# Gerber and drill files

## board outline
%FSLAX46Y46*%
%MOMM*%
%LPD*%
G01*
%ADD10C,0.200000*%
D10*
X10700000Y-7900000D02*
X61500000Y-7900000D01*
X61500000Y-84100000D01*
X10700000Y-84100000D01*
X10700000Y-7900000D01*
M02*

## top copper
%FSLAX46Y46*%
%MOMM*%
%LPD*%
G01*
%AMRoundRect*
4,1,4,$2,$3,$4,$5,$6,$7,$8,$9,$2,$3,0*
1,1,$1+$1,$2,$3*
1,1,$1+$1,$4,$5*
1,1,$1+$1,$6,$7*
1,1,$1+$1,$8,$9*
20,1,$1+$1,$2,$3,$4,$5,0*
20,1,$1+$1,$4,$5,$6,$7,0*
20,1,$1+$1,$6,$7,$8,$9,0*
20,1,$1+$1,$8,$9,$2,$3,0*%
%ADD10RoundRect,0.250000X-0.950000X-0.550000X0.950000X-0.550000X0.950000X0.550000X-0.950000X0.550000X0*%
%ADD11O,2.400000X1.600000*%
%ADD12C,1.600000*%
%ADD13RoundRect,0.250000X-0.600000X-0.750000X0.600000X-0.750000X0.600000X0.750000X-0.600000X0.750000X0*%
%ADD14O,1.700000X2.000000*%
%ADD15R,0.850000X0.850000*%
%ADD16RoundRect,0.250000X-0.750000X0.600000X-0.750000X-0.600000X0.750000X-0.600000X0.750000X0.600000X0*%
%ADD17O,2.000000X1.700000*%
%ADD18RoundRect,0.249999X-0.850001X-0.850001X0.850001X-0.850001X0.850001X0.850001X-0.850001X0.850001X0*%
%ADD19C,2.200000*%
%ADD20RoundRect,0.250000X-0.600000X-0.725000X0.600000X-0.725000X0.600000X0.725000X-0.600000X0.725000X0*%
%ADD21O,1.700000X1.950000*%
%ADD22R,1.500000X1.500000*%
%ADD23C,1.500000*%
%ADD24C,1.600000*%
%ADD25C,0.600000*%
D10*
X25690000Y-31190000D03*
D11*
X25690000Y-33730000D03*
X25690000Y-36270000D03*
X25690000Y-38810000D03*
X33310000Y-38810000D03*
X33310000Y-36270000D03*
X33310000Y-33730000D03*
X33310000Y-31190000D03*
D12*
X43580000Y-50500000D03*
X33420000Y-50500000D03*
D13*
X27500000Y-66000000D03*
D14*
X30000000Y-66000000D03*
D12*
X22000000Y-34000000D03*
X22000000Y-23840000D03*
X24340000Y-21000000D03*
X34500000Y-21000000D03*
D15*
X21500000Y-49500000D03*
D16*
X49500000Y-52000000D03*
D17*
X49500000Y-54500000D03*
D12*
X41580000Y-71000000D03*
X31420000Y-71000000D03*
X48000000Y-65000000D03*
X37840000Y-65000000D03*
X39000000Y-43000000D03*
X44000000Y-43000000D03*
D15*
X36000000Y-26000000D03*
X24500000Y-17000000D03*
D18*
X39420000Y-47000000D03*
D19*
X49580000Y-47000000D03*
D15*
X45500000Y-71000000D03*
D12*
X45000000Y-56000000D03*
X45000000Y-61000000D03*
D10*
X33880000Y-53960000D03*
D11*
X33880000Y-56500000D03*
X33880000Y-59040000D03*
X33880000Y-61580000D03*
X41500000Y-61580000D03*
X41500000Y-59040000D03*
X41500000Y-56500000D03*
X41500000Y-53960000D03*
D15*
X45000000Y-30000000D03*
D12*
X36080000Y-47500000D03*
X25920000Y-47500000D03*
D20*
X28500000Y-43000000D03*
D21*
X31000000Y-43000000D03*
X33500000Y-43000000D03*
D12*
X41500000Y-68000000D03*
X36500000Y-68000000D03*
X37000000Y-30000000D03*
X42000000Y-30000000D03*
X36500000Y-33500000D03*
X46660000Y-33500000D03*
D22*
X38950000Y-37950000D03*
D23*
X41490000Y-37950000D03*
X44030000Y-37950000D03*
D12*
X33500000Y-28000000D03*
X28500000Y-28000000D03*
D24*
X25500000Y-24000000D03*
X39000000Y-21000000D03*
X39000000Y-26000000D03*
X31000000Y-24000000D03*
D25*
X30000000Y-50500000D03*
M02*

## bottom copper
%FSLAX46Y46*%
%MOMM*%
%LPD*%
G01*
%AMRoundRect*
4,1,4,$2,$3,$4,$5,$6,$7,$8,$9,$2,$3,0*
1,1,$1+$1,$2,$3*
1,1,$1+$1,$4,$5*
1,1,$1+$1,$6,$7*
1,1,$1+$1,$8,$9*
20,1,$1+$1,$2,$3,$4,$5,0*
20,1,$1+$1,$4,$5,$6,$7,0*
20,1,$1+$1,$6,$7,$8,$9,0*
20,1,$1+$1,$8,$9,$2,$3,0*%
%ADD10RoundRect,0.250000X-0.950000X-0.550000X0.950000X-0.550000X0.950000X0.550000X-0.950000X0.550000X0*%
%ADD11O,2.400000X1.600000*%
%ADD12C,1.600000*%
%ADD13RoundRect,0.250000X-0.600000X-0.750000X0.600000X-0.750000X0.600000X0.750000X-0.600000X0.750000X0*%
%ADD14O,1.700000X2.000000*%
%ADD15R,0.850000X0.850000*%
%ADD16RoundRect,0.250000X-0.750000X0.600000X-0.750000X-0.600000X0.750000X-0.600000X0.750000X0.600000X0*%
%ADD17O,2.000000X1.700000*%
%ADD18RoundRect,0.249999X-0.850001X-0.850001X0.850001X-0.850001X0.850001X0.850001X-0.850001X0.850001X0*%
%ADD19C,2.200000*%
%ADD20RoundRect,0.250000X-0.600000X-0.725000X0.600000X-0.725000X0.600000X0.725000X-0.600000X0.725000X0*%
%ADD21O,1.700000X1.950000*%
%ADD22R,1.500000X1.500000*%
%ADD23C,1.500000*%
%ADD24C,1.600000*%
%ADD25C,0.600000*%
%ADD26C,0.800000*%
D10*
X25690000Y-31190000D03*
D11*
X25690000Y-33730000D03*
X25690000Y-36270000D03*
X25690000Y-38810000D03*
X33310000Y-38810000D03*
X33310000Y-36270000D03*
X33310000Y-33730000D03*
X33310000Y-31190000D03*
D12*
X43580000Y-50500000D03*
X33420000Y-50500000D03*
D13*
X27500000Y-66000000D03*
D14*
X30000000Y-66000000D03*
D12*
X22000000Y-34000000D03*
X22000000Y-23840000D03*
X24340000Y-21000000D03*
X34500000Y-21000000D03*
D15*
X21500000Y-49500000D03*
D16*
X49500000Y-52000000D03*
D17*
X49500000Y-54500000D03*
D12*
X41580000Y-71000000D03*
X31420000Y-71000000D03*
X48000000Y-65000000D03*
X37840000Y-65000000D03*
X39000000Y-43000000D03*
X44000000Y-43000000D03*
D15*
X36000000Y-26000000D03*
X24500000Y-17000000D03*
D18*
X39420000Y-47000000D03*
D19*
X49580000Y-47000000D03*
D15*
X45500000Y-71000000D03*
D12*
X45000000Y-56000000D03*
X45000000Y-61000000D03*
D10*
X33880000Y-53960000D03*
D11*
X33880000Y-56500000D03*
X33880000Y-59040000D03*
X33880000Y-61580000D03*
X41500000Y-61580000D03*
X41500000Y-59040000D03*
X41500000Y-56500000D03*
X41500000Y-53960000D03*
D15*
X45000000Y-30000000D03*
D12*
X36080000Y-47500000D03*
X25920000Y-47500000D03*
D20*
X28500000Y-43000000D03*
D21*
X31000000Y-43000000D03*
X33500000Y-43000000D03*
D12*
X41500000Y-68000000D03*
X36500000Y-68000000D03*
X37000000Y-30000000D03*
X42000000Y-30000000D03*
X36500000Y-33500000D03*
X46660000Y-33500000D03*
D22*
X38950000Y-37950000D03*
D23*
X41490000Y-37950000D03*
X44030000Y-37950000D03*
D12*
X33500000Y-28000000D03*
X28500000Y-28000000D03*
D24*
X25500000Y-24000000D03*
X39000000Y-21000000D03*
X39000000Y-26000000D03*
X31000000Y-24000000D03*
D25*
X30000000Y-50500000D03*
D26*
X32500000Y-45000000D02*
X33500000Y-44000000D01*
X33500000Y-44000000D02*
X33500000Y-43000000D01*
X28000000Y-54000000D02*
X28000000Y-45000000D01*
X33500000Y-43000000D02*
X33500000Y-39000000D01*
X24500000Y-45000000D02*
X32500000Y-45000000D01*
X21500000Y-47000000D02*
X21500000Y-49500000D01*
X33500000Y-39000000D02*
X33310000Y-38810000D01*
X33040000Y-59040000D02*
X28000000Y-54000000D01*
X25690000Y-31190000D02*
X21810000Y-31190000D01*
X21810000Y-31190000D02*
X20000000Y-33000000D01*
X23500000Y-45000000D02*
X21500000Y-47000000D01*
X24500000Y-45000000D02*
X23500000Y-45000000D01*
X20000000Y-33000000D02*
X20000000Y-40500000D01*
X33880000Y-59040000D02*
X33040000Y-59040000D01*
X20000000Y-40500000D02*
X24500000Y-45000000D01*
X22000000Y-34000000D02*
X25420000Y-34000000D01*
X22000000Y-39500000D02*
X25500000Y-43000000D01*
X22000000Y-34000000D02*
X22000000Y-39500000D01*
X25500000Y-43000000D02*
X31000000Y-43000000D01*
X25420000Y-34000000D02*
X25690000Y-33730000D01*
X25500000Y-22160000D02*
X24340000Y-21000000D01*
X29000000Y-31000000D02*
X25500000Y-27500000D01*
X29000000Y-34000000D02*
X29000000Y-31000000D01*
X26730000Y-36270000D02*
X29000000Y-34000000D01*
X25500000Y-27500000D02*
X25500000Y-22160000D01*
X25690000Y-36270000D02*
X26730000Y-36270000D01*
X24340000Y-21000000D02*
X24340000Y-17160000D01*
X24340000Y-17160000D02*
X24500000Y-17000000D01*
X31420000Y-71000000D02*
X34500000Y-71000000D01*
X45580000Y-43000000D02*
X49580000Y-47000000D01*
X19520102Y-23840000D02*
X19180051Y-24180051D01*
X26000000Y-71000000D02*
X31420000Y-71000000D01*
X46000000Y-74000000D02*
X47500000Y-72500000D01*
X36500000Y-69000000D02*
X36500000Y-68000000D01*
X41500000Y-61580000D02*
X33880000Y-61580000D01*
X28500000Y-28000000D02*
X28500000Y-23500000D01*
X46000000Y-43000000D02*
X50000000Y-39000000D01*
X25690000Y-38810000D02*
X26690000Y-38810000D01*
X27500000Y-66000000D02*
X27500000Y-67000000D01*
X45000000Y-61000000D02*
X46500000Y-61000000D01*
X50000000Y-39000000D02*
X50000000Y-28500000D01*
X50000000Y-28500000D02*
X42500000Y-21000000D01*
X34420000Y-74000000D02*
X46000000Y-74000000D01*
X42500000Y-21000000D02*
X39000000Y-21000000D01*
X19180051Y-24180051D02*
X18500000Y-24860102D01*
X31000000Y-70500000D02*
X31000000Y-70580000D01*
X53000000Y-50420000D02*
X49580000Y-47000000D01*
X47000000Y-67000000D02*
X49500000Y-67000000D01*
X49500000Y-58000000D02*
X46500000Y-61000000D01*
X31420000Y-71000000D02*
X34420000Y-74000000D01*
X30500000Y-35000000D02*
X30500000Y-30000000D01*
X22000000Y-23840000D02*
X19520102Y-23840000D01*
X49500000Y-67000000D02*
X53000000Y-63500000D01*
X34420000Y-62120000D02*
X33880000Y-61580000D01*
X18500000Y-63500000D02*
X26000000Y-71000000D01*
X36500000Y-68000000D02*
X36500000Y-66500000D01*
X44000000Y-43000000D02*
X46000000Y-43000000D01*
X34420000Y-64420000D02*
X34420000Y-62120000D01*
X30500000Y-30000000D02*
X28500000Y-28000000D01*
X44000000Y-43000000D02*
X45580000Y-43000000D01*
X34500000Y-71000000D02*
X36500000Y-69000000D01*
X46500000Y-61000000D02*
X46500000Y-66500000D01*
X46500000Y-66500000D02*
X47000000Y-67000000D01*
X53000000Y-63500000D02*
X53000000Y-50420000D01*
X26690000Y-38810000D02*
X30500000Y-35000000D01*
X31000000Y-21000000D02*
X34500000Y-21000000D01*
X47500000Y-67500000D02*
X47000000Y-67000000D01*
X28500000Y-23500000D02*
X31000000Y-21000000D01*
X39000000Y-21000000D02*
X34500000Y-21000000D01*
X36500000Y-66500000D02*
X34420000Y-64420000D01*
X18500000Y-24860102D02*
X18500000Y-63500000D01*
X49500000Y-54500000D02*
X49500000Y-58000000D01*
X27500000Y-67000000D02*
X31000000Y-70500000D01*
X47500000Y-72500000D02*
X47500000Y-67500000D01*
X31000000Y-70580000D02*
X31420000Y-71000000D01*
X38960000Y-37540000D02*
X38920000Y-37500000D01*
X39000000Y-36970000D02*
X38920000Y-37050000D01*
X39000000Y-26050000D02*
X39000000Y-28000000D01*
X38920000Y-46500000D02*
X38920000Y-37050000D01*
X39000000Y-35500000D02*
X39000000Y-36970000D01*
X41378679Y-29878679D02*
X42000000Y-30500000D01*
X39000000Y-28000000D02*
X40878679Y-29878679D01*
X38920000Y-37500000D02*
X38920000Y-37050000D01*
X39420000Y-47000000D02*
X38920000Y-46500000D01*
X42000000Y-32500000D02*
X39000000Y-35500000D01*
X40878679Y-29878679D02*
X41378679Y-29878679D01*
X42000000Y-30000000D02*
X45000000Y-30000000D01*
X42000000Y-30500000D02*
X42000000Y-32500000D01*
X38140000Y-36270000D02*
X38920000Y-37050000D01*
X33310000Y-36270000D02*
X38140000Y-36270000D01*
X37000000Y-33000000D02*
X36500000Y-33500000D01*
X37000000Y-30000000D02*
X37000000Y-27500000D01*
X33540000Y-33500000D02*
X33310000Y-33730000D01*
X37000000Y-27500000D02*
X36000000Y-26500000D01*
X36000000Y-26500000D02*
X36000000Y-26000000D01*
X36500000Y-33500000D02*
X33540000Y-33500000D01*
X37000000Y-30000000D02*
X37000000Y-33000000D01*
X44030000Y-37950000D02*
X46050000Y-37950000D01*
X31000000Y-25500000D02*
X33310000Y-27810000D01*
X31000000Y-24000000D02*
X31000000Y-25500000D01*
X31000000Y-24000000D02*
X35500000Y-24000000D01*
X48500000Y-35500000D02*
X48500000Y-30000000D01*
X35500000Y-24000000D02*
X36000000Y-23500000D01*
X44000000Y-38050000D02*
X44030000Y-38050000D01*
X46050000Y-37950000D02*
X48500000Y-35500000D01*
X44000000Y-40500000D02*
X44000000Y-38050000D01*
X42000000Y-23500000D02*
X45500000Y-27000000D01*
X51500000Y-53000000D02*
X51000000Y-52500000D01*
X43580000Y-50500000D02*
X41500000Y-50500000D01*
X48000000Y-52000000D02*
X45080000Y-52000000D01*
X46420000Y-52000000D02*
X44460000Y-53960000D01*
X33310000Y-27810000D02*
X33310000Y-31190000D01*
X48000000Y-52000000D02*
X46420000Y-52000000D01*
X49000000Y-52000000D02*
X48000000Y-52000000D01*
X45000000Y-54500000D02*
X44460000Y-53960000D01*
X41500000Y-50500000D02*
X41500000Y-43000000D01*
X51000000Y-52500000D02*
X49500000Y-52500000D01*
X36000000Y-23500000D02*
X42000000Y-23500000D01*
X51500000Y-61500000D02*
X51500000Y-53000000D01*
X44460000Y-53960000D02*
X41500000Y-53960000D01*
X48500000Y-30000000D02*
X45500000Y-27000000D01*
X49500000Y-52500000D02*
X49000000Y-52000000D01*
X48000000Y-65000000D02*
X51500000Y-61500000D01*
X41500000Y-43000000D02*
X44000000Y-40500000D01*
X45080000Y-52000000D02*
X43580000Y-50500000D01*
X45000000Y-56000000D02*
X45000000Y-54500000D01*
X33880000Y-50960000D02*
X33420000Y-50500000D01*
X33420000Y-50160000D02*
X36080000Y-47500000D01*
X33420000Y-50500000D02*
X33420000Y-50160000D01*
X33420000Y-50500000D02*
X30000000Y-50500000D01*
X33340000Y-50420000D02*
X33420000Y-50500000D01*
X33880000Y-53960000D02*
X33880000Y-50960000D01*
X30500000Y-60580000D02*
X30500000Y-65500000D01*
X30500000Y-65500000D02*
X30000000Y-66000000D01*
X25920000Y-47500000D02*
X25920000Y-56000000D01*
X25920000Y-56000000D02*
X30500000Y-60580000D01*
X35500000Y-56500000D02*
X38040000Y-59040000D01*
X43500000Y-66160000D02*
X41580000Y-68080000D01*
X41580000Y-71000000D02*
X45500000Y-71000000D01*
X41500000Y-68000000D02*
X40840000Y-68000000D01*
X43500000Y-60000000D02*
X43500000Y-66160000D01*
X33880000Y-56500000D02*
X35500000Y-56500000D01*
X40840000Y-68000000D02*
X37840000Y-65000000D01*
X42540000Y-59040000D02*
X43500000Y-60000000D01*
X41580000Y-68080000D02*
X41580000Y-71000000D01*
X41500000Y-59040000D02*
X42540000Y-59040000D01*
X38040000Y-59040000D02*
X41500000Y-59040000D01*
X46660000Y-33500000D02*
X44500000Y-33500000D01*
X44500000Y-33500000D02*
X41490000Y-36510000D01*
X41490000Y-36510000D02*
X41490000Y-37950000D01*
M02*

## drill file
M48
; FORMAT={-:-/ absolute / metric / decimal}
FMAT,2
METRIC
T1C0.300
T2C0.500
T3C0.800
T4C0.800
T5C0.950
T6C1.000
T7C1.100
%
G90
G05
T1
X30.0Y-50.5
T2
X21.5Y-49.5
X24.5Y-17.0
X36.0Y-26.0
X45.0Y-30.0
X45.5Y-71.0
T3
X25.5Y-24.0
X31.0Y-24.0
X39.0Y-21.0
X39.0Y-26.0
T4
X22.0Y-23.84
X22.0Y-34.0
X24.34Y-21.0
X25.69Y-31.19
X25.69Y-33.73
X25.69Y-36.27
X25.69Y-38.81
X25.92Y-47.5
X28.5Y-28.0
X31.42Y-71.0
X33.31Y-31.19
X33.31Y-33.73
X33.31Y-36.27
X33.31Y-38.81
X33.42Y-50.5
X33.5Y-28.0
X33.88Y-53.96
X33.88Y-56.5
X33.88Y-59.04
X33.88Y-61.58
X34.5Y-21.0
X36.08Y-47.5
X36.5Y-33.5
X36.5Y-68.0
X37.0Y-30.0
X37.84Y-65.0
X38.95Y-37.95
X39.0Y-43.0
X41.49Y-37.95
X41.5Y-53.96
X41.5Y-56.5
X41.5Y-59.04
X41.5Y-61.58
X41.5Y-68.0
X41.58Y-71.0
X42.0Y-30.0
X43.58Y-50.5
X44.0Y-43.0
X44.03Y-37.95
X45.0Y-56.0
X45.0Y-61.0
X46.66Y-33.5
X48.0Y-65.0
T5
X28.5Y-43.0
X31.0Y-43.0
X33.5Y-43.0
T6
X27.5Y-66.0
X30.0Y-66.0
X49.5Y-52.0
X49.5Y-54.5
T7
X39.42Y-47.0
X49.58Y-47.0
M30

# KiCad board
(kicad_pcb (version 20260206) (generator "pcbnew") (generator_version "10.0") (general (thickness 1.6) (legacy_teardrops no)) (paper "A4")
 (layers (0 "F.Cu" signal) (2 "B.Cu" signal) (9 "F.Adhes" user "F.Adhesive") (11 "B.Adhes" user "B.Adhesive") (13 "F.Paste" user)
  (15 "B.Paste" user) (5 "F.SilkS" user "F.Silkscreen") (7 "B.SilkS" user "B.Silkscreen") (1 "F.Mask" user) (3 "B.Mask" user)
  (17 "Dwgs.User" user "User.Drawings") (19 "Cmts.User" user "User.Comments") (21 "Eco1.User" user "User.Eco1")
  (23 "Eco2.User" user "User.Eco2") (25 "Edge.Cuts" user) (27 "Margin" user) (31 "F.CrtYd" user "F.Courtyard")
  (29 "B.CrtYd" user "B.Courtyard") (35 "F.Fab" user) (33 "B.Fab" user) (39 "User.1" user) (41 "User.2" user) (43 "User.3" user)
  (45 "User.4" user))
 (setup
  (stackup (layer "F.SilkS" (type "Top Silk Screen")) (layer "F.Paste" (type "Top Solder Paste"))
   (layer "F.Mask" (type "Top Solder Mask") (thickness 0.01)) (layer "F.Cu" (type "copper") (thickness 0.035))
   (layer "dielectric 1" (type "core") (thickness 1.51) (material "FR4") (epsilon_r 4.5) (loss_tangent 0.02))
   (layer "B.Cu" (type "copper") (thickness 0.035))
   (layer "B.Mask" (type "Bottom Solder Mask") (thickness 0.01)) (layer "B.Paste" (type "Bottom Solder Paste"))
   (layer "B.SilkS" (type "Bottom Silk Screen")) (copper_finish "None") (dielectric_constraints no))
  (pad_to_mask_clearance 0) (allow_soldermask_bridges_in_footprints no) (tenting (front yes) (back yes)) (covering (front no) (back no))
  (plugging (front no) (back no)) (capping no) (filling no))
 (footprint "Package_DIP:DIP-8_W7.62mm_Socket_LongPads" (layer "F.Cu") (at 25.69 31.19)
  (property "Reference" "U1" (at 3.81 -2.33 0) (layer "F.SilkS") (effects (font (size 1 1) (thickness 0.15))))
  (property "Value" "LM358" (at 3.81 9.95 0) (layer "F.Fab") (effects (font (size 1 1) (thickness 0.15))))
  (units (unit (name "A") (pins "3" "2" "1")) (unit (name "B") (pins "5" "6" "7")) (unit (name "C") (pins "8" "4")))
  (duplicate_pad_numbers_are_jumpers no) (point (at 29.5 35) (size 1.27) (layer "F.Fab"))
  (pad "1" thru_hole roundrect (at 0 0) (size 2.4 1.6) (drill 0.8) (layers "*.Cu" "*.Mask") (remove_unused_layers no)
   (roundrect_rratio 0.15625) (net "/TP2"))
  (pad "2" thru_hole oval (at 0 2.54) (size 2.4 1.6) (drill 0.8) (layers "*.Cu" "*.Mask") (remove_unused_layers no) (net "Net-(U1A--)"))
  (pad "3" thru_hole oval (at 0 5.08) (size 2.4 1.6) (drill 0.8) (layers "*.Cu" "*.Mask") (remove_unused_layers no) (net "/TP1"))
  (pad "4" thru_hole oval (at 0 7.62) (size 2.4 1.6) (drill 0.8) (layers "*.Cu" "*.Mask") (remove_unused_layers no) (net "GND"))
  (pad "5" thru_hole oval (at 7.62 7.62) (size 2.4 1.6) (drill 0.8) (layers "*.Cu" "*.Mask") (remove_unused_layers no) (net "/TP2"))
  (pad "6" thru_hole oval (at 7.62 5.08) (size 2.4 1.6) (drill 0.8) (layers "*.Cu" "*.Mask") (remove_unused_layers no) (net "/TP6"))
  (pad "7" thru_hole oval (at 7.62 2.54) (size 2.4 1.6) (drill 0.8) (layers "*.Cu" "*.Mask") (remove_unused_layers no) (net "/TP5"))
  (pad "8" thru_hole oval (at 7.62 0) (size 2.4 1.6) (drill 0.8) (layers "*.Cu" "*.Mask") (remove_unused_layers no) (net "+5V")))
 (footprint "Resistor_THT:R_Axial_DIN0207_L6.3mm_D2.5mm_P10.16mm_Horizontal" (layer "F.Cu") (at 43.58 50.5 180)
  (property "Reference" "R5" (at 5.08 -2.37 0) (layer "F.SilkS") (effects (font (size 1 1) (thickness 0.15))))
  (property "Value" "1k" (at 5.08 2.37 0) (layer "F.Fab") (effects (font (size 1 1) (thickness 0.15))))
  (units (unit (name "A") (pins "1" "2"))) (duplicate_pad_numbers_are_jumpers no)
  (pad "1" thru_hole circle (at 0 0 180) (size 1.6 1.6) (drill 0.8) (layers "*.Cu" "*.Mask") (remove_unused_layers no) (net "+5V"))
  (pad "2" thru_hole circle (at 10.16 0 180) (size 1.6 1.6) (drill 0.8) (layers "*.Cu" "*.Mask") (remove_unused_layers no) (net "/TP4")))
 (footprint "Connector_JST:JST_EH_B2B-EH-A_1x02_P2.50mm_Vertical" (layer "F.Cu") (at 27.5 66)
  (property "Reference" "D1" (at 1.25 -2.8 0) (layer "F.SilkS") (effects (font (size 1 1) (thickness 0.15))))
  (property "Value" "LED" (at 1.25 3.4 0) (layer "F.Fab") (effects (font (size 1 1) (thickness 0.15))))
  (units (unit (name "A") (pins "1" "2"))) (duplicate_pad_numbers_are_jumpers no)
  (pad "1" thru_hole roundrect (at 0 0) (size 1.7 2) (drill 1) (layers "*.Cu" "*.Mask") (remove_unused_layers no)
   (roundrect_rratio 0.147059) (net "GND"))
  (pad "2" thru_hole oval (at 2.5 0) (size 1.7 2) (drill 1) (layers "*.Cu" "*.Mask") (remove_unused_layers no) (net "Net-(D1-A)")))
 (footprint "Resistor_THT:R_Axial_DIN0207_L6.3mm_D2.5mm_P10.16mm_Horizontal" (layer "F.Cu") (at 22 34 90)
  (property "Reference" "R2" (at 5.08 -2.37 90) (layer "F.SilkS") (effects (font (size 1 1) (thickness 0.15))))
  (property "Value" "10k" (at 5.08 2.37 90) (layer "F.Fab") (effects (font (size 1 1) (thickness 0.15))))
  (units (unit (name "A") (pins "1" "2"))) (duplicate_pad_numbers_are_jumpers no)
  (pad "1" thru_hole circle (at 0 0 90) (size 1.6 1.6) (drill 0.8) (layers "*.Cu" "*.Mask") (remove_unused_layers no) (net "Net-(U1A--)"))
  (pad "2" thru_hole circle (at 10.16 0 90) (size 1.6 1.6) (drill 0.8) (layers "*.Cu" "*.Mask") (remove_unused_layers no) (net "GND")))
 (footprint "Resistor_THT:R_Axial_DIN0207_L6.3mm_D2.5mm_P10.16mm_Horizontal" (layer "F.Cu") (at 24.34 21)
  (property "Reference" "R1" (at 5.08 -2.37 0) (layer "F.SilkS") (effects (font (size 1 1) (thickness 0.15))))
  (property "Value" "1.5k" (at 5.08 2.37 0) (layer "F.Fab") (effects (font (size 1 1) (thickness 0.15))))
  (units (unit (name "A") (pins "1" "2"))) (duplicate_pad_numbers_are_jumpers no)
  (pad "1" thru_hole circle (at 0 0) (size 1.6 1.6) (drill 0.8) (layers "*.Cu" "*.Mask") (remove_unused_layers no) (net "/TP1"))
  (pad "2" thru_hole circle (at 10.16 0) (size 1.6 1.6) (drill 0.8) (layers "*.Cu" "*.Mask") (remove_unused_layers no) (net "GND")))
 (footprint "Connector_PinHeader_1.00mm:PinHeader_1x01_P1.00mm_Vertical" (layer "F.Cu") (at 21.5 49.5)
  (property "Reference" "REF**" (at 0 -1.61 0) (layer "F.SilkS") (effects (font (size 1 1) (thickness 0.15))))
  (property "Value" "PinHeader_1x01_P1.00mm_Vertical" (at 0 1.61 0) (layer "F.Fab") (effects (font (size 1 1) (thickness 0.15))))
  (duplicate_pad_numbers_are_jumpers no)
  (pad "1" thru_hole rect (at 0 0) (size 0.85 0.85) (drill 0.5) (layers "*.Cu" "*.Mask") (remove_unused_layers no) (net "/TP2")))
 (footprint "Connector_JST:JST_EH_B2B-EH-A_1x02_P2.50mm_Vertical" (layer "F.Cu") (at 49.5 52 -90)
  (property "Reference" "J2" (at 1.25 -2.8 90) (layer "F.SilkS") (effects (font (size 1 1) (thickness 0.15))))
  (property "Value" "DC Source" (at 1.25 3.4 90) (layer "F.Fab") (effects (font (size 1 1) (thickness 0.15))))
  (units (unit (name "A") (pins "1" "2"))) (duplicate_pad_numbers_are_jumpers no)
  (pad "1" thru_hole roundrect (at 0 0 270) (size 1.7 2) (drill 1) (layers "*.Cu" "*.Mask") (remove_unused_layers no)
   (roundrect_rratio 0.147059) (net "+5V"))
  (pad "2" thru_hole oval (at 2.5 0 270) (size 1.7 2) (drill 1) (layers "*.Cu" "*.Mask") (remove_unused_layers no) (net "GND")))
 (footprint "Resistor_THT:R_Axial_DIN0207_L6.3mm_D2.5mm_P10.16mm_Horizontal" (layer "F.Cu") (at 41.58 71 180)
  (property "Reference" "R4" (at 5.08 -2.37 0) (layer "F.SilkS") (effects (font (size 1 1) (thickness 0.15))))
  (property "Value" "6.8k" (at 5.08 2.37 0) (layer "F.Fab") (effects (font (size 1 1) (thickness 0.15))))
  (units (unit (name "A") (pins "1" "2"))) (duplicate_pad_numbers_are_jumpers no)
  (pad "1" thru_hole circle (at 0 0 180) (size 1.6 1.6) (drill 0.8) (layers "*.Cu" "*.Mask") (remove_unused_layers no) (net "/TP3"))
  (pad "2" thru_hole circle (at 10.16 0 180) (size 1.6 1.6) (drill 0.8) (layers "*.Cu" "*.Mask") (remove_unused_layers no) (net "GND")))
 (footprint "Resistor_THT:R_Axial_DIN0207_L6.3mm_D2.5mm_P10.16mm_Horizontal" (layer "F.Cu") (at 48 65 180)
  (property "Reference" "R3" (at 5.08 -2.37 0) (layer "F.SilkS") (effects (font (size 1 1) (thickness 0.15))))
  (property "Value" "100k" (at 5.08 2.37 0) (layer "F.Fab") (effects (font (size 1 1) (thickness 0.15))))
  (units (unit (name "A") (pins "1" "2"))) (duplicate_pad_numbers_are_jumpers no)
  (pad "1" thru_hole circle (at 0 0 180) (size 1.6 1.6) (drill 0.8) (layers "*.Cu" "*.Mask") (remove_unused_layers no) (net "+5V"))
  (pad "2" thru_hole circle (at 10.16 0 180) (size 1.6 1.6) (drill 0.8) (layers "*.Cu" "*.Mask") (remove_unused_layers no) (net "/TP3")))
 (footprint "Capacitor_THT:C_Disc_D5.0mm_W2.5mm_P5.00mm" (layer "F.Cu") (at 39 43)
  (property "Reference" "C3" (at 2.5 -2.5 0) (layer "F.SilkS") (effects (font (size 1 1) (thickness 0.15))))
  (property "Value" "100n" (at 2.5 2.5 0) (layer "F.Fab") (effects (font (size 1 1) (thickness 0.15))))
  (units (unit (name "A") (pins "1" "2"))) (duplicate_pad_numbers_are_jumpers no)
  (pad "1" thru_hole circle (at 0 0) (size 1.6 1.6) (drill 0.8) (layers "*.Cu" "*.Mask") (remove_unused_layers no) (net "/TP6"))
  (pad "2" thru_hole circle (at 5 0) (size 1.6 1.6) (drill 0.8) (layers "*.Cu" "*.Mask") (remove_unused_layers no) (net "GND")))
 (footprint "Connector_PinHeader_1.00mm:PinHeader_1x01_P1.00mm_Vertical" (layer "F.Cu") (at 36 26)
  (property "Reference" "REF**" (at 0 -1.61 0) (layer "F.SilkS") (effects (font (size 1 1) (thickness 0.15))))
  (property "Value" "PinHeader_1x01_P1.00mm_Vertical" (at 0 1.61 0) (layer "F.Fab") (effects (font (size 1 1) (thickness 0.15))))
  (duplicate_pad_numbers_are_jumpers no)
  (pad "1" thru_hole rect (at 0 0) (size 0.85 0.85) (drill 0.5) (layers "*.Cu" "*.Mask") (remove_unused_layers no) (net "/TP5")))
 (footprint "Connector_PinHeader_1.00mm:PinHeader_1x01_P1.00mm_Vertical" (layer "F.Cu") (at 24.5 17)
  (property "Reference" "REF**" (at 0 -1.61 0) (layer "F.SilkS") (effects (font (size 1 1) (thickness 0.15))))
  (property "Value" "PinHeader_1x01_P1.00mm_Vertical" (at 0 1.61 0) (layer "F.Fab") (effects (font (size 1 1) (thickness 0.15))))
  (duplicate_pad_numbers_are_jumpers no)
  (pad "1" thru_hole rect (at 0 0) (size 0.85 0.85) (drill 0.5) (layers "*.Cu" "*.Mask") (remove_unused_layers no) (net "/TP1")))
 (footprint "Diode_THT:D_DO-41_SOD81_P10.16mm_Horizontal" (layer "F.Cu") (at 39.42 47)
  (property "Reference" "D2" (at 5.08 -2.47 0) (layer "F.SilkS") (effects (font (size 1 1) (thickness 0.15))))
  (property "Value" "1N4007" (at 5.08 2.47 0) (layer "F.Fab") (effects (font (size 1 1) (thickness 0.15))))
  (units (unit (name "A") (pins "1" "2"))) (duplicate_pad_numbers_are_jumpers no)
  (pad "1" thru_hole roundrect (at 0 0) (size 2.2 2.2) (drill 1.1) (layers "*.Cu" "*.Mask") (remove_unused_layers no)
   (roundrect_rratio 0.113636) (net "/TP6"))
  (pad "2" thru_hole circle (at 10.16 0) (size 2.2 2.2) (drill 1.1) (layers "*.Cu" "*.Mask") (remove_unused_layers no) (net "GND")))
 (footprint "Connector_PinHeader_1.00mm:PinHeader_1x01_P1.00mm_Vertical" (layer "F.Cu") (at 45.5 71)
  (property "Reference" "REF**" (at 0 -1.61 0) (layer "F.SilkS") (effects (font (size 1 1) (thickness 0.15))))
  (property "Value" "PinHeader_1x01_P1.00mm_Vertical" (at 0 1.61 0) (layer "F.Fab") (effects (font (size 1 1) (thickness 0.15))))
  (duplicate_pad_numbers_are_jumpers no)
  (pad "1" thru_hole rect (at 0 0) (size 0.85 0.85) (drill 0.5) (layers "*.Cu" "*.Mask") (remove_unused_layers no) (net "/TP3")))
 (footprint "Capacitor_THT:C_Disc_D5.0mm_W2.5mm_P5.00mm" (layer "F.Cu") (at 45 56 -90)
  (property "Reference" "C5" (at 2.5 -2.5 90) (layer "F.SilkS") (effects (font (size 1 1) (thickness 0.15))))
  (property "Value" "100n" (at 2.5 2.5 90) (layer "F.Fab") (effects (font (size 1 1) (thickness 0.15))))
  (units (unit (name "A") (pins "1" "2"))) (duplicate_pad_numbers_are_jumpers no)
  (pad "1" thru_hole circle (at 0 0 270) (size 1.6 1.6) (drill 0.8) (layers "*.Cu" "*.Mask") (remove_unused_layers no) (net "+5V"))
  (pad "2" thru_hole circle (at 5 0 270) (size 1.6 1.6) (drill 0.8) (layers "*.Cu" "*.Mask") (remove_unused_layers no) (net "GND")))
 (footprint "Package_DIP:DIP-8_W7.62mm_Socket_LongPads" (layer "F.Cu") (at 33.88 53.96)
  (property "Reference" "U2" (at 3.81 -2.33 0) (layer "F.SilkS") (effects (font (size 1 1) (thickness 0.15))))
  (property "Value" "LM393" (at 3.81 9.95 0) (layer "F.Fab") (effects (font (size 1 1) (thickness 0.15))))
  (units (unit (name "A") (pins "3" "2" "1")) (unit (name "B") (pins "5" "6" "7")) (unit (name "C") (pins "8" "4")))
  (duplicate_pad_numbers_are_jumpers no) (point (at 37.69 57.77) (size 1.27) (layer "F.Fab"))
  (pad "1" thru_hole roundrect (at 0 0) (size 2.4 1.6) (drill 0.8) (layers "*.Cu" "*.Mask") (remove_unused_layers no)
   (roundrect_rratio 0.15625) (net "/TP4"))
  (pad "2" thru_hole oval (at 0 2.54) (size 2.4 1.6) (drill 0.8) (layers "*.Cu" "*.Mask") (remove_unused_layers no) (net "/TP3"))
  (pad "3" thru_hole oval (at 0 5.08) (size 2.4 1.6) (drill 0.8) (layers "*.Cu" "*.Mask") (remove_unused_layers no) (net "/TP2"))
  (pad "4" thru_hole oval (at 0 7.62) (size 2.4 1.6) (drill 0.8) (layers "*.Cu" "*.Mask") (remove_unused_layers no) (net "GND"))
  (pad "5" thru_hole oval (at 7.62 7.62) (size 2.4 1.6) (drill 0.8) (layers "*.Cu" "*.Mask") (remove_unused_layers no) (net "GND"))
  (pad "6" thru_hole oval (at 7.62 5.08) (size 2.4 1.6) (drill 0.8) (layers "*.Cu" "*.Mask") (remove_unused_layers no) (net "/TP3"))
  (pad "7" thru_hole oval (at 7.62 2.54) (size 2.4 1.6) (drill 0.8) (layers "*.Cu" "*.Mask") (remove_unused_layers no)
   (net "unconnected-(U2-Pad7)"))
  (pad "8" thru_hole oval (at 7.62 0) (size 2.4 1.6) (drill 0.8) (layers "*.Cu" "*.Mask") (remove_unused_layers no) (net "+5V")))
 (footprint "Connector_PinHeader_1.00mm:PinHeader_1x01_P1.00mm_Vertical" (layer "F.Cu") (at 45 30)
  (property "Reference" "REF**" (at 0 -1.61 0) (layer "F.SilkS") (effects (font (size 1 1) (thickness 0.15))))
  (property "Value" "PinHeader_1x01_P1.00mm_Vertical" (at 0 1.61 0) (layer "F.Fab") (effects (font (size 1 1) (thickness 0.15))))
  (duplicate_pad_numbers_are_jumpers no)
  (pad "1" thru_hole rect (at 0 0) (size 0.85 0.85) (drill 0.5) (layers "*.Cu" "*.Mask") (remove_unused_layers no) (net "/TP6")))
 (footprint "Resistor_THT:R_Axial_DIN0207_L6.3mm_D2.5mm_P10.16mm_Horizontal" (layer "F.Cu") (at 36.08 47.5 180)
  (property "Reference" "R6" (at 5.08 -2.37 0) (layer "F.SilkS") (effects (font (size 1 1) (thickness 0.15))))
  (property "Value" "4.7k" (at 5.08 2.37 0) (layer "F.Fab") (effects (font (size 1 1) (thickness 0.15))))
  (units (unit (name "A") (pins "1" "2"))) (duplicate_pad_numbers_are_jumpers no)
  (pad "1" thru_hole circle (at 0 0 180) (size 1.6 1.6) (drill 0.8) (layers "*.Cu" "*.Mask") (remove_unused_layers no) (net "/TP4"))
  (pad "2" thru_hole circle (at 10.16 0 180) (size 1.6 1.6) (drill 0.8) (layers "*.Cu" "*.Mask") (remove_unused_layers no)
   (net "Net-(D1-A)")))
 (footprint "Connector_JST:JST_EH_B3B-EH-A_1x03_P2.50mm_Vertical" (layer "F.Cu") (at 28.5 43)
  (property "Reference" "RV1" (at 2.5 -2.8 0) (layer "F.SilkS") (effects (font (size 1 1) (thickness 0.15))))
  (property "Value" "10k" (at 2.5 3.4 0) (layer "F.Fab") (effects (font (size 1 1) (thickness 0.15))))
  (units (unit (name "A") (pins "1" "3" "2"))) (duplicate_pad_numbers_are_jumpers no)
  (pad "1" thru_hole roundrect (at 0 0) (size 1.7 1.95) (drill 0.95) (layers "*.Cu" "*.Mask") (remove_unused_layers no)
   (roundrect_rratio 0.147059) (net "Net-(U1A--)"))
  (pad "2" thru_hole oval (at 2.5 0) (size 1.7 1.95) (drill 0.95) (layers "*.Cu" "*.Mask") (remove_unused_layers no) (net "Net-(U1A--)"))
  (pad "3" thru_hole oval (at 5 0) (size 1.7 1.95) (drill 0.95) (layers "*.Cu" "*.Mask") (remove_unused_layers no) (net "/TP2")))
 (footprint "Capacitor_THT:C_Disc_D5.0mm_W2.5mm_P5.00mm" (layer "F.Cu") (at 41.5 68 180)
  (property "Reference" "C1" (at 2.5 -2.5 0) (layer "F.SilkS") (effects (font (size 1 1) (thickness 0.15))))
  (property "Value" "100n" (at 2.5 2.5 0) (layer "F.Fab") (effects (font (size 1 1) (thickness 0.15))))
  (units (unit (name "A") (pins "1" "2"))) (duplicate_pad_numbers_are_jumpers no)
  (pad "1" thru_hole circle (at 0 0 180) (size 1.6 1.6) (drill 0.8) (layers "*.Cu" "*.Mask") (remove_unused_layers no) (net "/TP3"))
  (pad "2" thru_hole circle (at 5 0 180) (size 1.6 1.6) (drill 0.8) (layers "*.Cu" "*.Mask") (remove_unused_layers no) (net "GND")))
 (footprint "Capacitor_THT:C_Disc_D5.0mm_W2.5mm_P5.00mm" (layer "F.Cu") (at 37 30)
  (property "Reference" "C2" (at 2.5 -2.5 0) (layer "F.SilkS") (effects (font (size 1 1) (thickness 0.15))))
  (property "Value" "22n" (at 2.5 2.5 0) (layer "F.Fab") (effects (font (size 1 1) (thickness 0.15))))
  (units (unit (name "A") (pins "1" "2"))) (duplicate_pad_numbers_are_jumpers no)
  (pad "1" thru_hole circle (at 0 0) (size 1.6 1.6) (drill 0.8) (layers "*.Cu" "*.Mask") (remove_unused_layers no) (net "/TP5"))
  (pad "2" thru_hole circle (at 5 0) (size 1.6 1.6) (drill 0.8) (layers "*.Cu" "*.Mask") (remove_unused_layers no) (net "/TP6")))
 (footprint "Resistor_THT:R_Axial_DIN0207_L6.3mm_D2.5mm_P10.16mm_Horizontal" (layer "F.Cu") (at 36.5 33.5)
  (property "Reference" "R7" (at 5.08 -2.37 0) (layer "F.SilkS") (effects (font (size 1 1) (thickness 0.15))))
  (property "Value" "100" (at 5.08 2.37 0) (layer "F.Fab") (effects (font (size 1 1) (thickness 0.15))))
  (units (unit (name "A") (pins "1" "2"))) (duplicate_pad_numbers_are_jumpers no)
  (pad "1" thru_hole circle (at 0 0) (size 1.6 1.6) (drill 0.8) (layers "*.Cu" "*.Mask") (remove_unused_layers no) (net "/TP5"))
  (pad "2" thru_hole circle (at 10.16 0) (size 1.6 1.6) (drill 0.8) (layers "*.Cu" "*.Mask") (remove_unused_layers no) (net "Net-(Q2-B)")))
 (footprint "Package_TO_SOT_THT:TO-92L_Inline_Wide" (layer "F.Cu") (at 38.95 37.95)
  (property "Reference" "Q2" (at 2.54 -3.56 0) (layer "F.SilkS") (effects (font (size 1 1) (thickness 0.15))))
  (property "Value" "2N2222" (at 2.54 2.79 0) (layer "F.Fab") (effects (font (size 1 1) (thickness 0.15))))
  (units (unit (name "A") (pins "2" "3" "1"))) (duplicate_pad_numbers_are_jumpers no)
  (pad "1" thru_hole rect (at 0 0) (size 1.5 1.5) (drill 0.8) (layers "*.Cu" "*.Mask") (remove_unused_layers no) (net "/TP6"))
  (pad "2" thru_hole circle (at 2.54 0) (size 1.5 1.5) (drill 0.8) (layers "*.Cu" "*.Mask") (remove_unused_layers no) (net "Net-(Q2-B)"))
  (pad "3" thru_hole circle (at 5.08 0) (size 1.5 1.5) (drill 0.8) (layers "*.Cu" "*.Mask") (remove_unused_layers no) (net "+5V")))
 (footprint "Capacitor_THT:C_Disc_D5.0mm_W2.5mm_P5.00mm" (layer "F.Cu") (at 33.5 28 180)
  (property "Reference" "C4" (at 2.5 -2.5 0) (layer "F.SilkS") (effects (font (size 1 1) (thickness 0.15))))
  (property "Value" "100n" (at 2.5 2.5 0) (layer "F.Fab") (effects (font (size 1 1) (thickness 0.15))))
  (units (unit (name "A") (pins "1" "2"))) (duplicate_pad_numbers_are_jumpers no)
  (pad "1" thru_hole circle (at 0 0 180) (size 1.6 1.6) (drill 0.8) (layers "*.Cu" "*.Mask") (remove_unused_layers no) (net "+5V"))
  (pad "2" thru_hole circle (at 5 0 180) (size 1.6 1.6) (drill 0.8) (layers "*.Cu" "*.Mask") (remove_unused_layers no) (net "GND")))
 (gr_rect (start 10.7 7.9) (end 61.5 84.1) (stroke (width 0.2) (type solid)) (fill no) (layer "Edge.Cuts"))
 (segment (start 32.5 45) (end 33.5 44) (width 0.8) (layer "B.Cu") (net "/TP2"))
 (segment (start 33.5 44) (end 33.5 43) (width 0.8) (layer "B.Cu") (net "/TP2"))
 (segment (start 28 54) (end 28 45) (width 0.8) (layer "B.Cu") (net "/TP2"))
 (segment (start 33.5 43) (end 33.5 39) (width 0.8) (layer "B.Cu") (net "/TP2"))
 (segment (start 24.5 45) (end 32.5 45) (width 0.8) (layer "B.Cu") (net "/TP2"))
 (segment (start 21.5 47) (end 21.5 49.5) (width 0.8) (layer "B.Cu") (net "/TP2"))
 (segment (start 33.5 39) (end 33.31 38.81) (width 0.8) (layer "B.Cu") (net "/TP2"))
 (segment (start 33.04 59.04) (end 28 54) (width 0.8) (layer "B.Cu") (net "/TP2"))
 (segment (start 25.69 31.19) (end 21.81 31.19) (width 0.8) (layer "B.Cu") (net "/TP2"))
 (segment (start 21.81 31.19) (end 20 33) (width 0.8) (layer "B.Cu") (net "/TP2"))
 (segment (start 23.5 45) (end 21.5 47) (width 0.8) (layer "B.Cu") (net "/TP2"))
 (segment (start 24.5 45) (end 23.5 45) (width 0.8) (layer "B.Cu") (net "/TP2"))
 (segment (start 20 33) (end 20 40.5) (width 0.8) (layer "B.Cu") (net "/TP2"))
 (segment (start 33.88 59.04) (end 33.04 59.04) (width 0.8) (layer "B.Cu") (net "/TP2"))
 (segment (start 20 40.5) (end 24.5 45) (width 0.8) (layer "B.Cu") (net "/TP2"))
 (segment (start 22 34) (end 25.42 34) (width 0.8) (layer "B.Cu") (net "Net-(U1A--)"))
 (segment (start 22 39.5) (end 25.5 43) (width 0.8) (layer "B.Cu") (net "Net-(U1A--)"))
 (segment (start 22 34) (end 22 39.5) (width 0.8) (layer "B.Cu") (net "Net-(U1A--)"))
 (segment (start 25.5 43) (end 31 43) (width 0.8) (layer "B.Cu") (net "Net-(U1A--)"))
 (segment (start 25.42 34) (end 25.69 33.73) (width 0.8) (layer "B.Cu") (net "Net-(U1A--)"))
 (via (at 25.5 24) (size 1.6) (drill 0.8) (layers "F.Cu" "B.Cu") (free yes) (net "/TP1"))
 (segment (start 25.5 22.16) (end 24.34 21) (width 0.8) (layer "B.Cu") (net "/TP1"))
 (segment (start 29 31) (end 25.5 27.5) (width 0.8) (layer "B.Cu") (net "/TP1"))
 (segment (start 29 34) (end 29 31) (width 0.8) (layer "B.Cu") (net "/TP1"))
 (segment (start 26.73 36.27) (end 29 34) (width 0.8) (layer "B.Cu") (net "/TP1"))
 (segment (start 25.5 27.5) (end 25.5 22.16) (width 0.8) (layer "B.Cu") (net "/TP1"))
 (segment (start 25.69 36.27) (end 26.73 36.27) (width 0.8) (layer "B.Cu") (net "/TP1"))
 (segment (start 24.34 21) (end 24.34 17.16) (width 0.8) (layer "B.Cu") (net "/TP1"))
 (segment (start 24.34 17.16) (end 24.5 17) (width 0.8) (layer "B.Cu") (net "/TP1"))
 (via (at 39 21) (size 1.6) (drill 0.8) (layers "F.Cu" "B.Cu") (free yes) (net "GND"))
 (segment (start 31.42 71) (end 34.5 71) (width 0.8) (layer "B.Cu") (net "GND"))
 (segment (start 45.58 43) (end 49.58 47) (width 0.8) (layer "B.Cu") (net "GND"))
 (segment (start 19.520102 23.84) (end 19.180051 24.180051) (width 0.8) (layer "B.Cu") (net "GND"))
 (segment (start 26 71) (end 31.42 71) (width 0.8) (layer "B.Cu") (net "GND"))
 (segment (start 46 74) (end 47.5 72.5) (width 0.8) (layer "B.Cu") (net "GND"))
 (segment (start 36.5 69) (end 36.5 68) (width 0.8) (layer "B.Cu") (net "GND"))
 (segment (start 41.5 61.58) (end 33.88 61.58) (width 0.8) (layer "B.Cu") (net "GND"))
 (segment (start 28.5 28) (end 28.5 23.5) (width 0.8) (layer "B.Cu") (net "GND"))
 (segment (start 46 43) (end 50 39) (width 0.8) (layer "B.Cu") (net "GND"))
 (segment (start 25.69 38.81) (end 26.69 38.81) (width 0.8) (layer "B.Cu") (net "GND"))
 (segment (start 27.5 66) (end 27.5 67) (width 0.8) (layer "B.Cu") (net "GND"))
 (segment (start 45 61) (end 46.5 61) (width 0.8) (layer "B.Cu") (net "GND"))
 (segment (start 50 39) (end 50 28.5) (width 0.8) (layer "B.Cu") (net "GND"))
 (segment (start 50 28.5) (end 42.5 21) (width 0.8) (layer "B.Cu") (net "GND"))
 (segment (start 34.42 74) (end 46 74) (width 0.8) (layer "B.Cu") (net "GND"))
 (segment (start 42.5 21) (end 39 21) (width 0.8) (layer "B.Cu") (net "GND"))
 (segment (start 19.180051 24.180051) (end 18.5 24.860102) (width 0.8) (layer "B.Cu") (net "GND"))
 (segment (start 31 70.5) (end 31 70.58) (width 0.8) (layer "B.Cu") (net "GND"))
 (segment (start 53 50.42) (end 49.58 47) (width 0.8) (layer "B.Cu") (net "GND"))
 (segment (start 47 67) (end 49.5 67) (width 0.8) (layer "B.Cu") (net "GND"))
 (segment (start 49.5 58) (end 46.5 61) (width 0.8) (layer "B.Cu") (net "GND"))
 (segment (start 31.42 71) (end 34.42 74) (width 0.8) (layer "B.Cu") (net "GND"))
 (segment (start 30.5 35) (end 30.5 30) (width 0.8) (layer "B.Cu") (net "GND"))
 (segment (start 22 23.84) (end 19.520102 23.84) (width 0.8) (layer "B.Cu") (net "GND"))
 (segment (start 49.5 67) (end 53 63.5) (width 0.8) (layer "B.Cu") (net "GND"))
 (segment (start 34.42 62.12) (end 33.88 61.58) (width 0.8) (layer "B.Cu") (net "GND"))
 (segment (start 18.5 63.5) (end 26 71) (width 0.8) (layer "B.Cu") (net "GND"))
 (segment (start 36.5 68) (end 36.5 66.5) (width 0.8) (layer "B.Cu") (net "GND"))
 (segment (start 44 43) (end 46 43) (width 0.8) (layer "B.Cu") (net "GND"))
 (segment (start 34.42 64.42) (end 34.42 62.12) (width 0.8) (layer "B.Cu") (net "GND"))
 (segment (start 30.5 30) (end 28.5 28) (width 0.8) (layer "B.Cu") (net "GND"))
 (segment (start 44 43) (end 45.58 43) (width 0.8) (layer "B.Cu") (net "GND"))
 (segment (start 34.5 71) (end 36.5 69) (width 0.8) (layer "B.Cu") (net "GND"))
 (segment (start 46.5 61) (end 46.5 66.5) (width 0.8) (layer "B.Cu") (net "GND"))
 (segment (start 46.5 66.5) (end 47 67) (width 0.8) (layer "B.Cu") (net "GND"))
 (segment (start 53 63.5) (end 53 50.42) (width 0.8) (layer "B.Cu") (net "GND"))
 (segment (start 26.69 38.81) (end 30.5 35) (width 0.8) (layer "B.Cu") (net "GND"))
 (segment (start 31 21) (end 34.5 21) (width 0.8) (layer "B.Cu") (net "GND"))
 (segment (start 47.5 67.5) (end 47 67) (width 0.8) (layer "B.Cu") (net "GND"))
 (segment (start 28.5 23.5) (end 31 21) (width 0.8) (layer "B.Cu") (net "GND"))
 (segment (start 39 21) (end 34.5 21) (width 0.8) (layer "B.Cu") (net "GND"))
 (segment (start 36.5 66.5) (end 34.42 64.42) (width 0.8) (layer "B.Cu") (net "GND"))
 (segment (start 18.5 24.860102) (end 18.5 63.5) (width 0.8) (layer "B.Cu") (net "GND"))
 (segment (start 49.5 54.5) (end 49.5 58) (width 0.8) (layer "B.Cu") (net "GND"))
 (segment (start 27.5 67) (end 31 70.5) (width 0.8) (layer "B.Cu") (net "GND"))
 (segment (start 47.5 72.5) (end 47.5 67.5) (width 0.8) (layer "B.Cu") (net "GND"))
 (segment (start 31 70.58) (end 31.42 71) (width 0.8) (layer "B.Cu") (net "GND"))
 (via (at 39 26) (size 1.6) (drill 0.8) (layers "F.Cu" "B.Cu") (free yes) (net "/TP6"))
 (segment (start 38.96 37.54) (end 38.92 37.5) (width 0.8) (layer "B.Cu") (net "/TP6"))
 (segment (start 39 36.97) (end 38.92 37.05) (width 0.8) (layer "B.Cu") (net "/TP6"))
 (segment (start 39 26.05) (end 39 28) (width 0.8) (layer "B.Cu") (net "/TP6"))
 (segment (start 38.92 46.5) (end 38.92 37.05) (width 0.8) (layer "B.Cu") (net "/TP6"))
 (segment (start 39 35.5) (end 39 36.97) (width 0.8) (layer "B.Cu") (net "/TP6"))
 (segment (start 41.378679 29.878679) (end 42 30.5) (width 0.8) (layer "B.Cu") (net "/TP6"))
 (segment (start 39 28) (end 40.878679 29.878679) (width 0.8) (layer "B.Cu") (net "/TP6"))
 (segment (start 38.92 37.5) (end 38.92 37.05) (width 0.8) (layer "B.Cu") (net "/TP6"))
 (segment (start 39.42 47) (end 38.92 46.5) (width 0.8) (layer "B.Cu") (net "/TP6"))
 (segment (start 42 32.5) (end 39 35.5) (width 0.8) (layer "B.Cu") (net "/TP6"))
 (segment (start 40.878679 29.878679) (end 41.378679 29.878679) (width 0.8) (layer "B.Cu") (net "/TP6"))
 (segment (start 42 30) (end 45 30) (width 0.8) (layer "B.Cu") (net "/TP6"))
 (segment (start 42 30.5) (end 42 32.5) (width 0.8) (layer "B.Cu") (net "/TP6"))
 (segment (start 38.14 36.27) (end 38.92 37.05) (width 0.8) (layer "B.Cu") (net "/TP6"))
 (segment (start 33.31 36.27) (end 38.14 36.27) (width 0.8) (layer "B.Cu") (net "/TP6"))
 (segment (start 37 33) (end 36.5 33.5) (width 0.8) (layer "B.Cu") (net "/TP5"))
 (segment (start 37 30) (end 37 27.5) (width 0.8) (layer "B.Cu") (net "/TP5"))
 (segment (start 33.54 33.5) (end 33.31 33.73) (width 0.8) (layer "B.Cu") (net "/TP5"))
 (segment (start 37 27.5) (end 36 26.5) (width 0.8) (layer "B.Cu") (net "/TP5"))
 (segment (start 36 26.5) (end 36 26) (width 0.8) (layer "B.Cu") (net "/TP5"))
 (segment (start 36.5 33.5) (end 33.54 33.5) (width 0.8) (layer "B.Cu") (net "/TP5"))
 (segment (start 37 30) (end 37 33) (width 0.8) (layer "B.Cu") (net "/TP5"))
 (via (at 31 24) (size 1.6) (drill 0.8) (layers "F.Cu" "B.Cu") (free yes) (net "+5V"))
 (segment (start 44.03 37.95) (end 46.05 37.95) (width 0.8) (layer "B.Cu") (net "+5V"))
 (segment (start 31 25.5) (end 33.31 27.81) (width 0.8) (layer "B.Cu") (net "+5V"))
 (segment (start 31 24) (end 31 25.5) (width 0.8) (layer "B.Cu") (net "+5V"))
 (segment (start 31 24) (end 35.5 24) (width 0.8) (layer "B.Cu") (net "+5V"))
 (segment (start 48.5 35.5) (end 48.5 30) (width 0.8) (layer "B.Cu") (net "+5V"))
 (segment (start 35.5 24) (end 36 23.5) (width 0.8) (layer "B.Cu") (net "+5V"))
 (segment (start 44 38.05) (end 44.03 38.05) (width 0.8) (layer "B.Cu") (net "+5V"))
 (segment (start 46.05 37.95) (end 48.5 35.5) (width 0.8) (layer "B.Cu") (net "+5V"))
 (segment (start 44 40.5) (end 44 38.05) (width 0.8) (layer "B.Cu") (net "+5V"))
 (segment (start 42 23.5) (end 45.5 27) (width 0.8) (layer "B.Cu") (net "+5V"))
 (segment (start 51.5 53) (end 51 52.5) (width 0.8) (layer "B.Cu") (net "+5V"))
 (segment (start 43.58 50.5) (end 41.5 50.5) (width 0.8) (layer "B.Cu") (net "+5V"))
 (segment (start 48 52) (end 45.08 52) (width 0.8) (layer "B.Cu") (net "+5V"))
 (segment (start 46.42 52) (end 44.46 53.96) (width 0.8) (layer "B.Cu") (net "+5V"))
 (segment (start 33.31 27.81) (end 33.31 31.19) (width 0.8) (layer "B.Cu") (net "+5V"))
 (segment (start 48 52) (end 46.42 52) (width 0.8) (layer "B.Cu") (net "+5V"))
 (segment (start 49 52) (end 48 52) (width 0.8) (layer "B.Cu") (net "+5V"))
 (segment (start 45 54.5) (end 44.46 53.96) (width 0.8) (layer "B.Cu") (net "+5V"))
 (segment (start 41.5 50.5) (end 41.5 43) (width 0.8) (layer "B.Cu") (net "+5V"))
 (segment (start 51 52.5) (end 49.5 52.5) (width 0.8) (layer "B.Cu") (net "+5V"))
 (segment (start 36 23.5) (end 42 23.5) (width 0.8) (layer "B.Cu") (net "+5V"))
 (segment (start 51.5 61.5) (end 51.5 53) (width 0.8) (layer "B.Cu") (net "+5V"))
 (segment (start 44.46 53.96) (end 41.5 53.96) (width 0.8) (layer "B.Cu") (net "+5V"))
 (segment (start 48.5 30) (end 45.5 27) (width 0.8) (layer "B.Cu") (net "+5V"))
 (segment (start 49.5 52.5) (end 49 52) (width 0.8) (layer "B.Cu") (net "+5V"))
 (segment (start 48 65) (end 51.5 61.5) (width 0.8) (layer "B.Cu") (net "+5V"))
 (segment (start 41.5 43) (end 44 40.5) (width 0.8) (layer "B.Cu") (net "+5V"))
 (segment (start 45.08 52) (end 43.58 50.5) (width 0.8) (layer "B.Cu") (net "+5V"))
 (segment (start 45 56) (end 45 54.5) (width 0.8) (layer "B.Cu") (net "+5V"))
 (via (at 30 50.5) (size 0.6) (drill 0.3) (layers "F.Cu" "B.Cu") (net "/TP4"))
 (segment (start 33.88 50.96) (end 33.42 50.5) (width 0.8) (layer "B.Cu") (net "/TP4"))
 (segment (start 33.42 50.16) (end 36.08 47.5) (width 0.8) (layer "B.Cu") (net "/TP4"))
 (segment (start 33.42 50.5) (end 33.42 50.16) (width 0.8) (layer "B.Cu") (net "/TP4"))
 (segment (start 33.42 50.5) (end 30 50.5) (width 0.8) (layer "B.Cu") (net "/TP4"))
 (segment (start 33.34 50.42) (end 33.42 50.5) (width 0.8) (layer "B.Cu") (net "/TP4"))
 (segment (start 33.88 53.96) (end 33.88 50.96) (width 0.8) (layer "B.Cu") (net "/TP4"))
 (segment (start 30.5 60.58) (end 30.5 65.5) (width 0.8) (layer "B.Cu") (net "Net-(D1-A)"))
 (segment (start 30.5 65.5) (end 30 66) (width 0.8) (layer "B.Cu") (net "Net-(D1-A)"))
 (segment (start 25.92 47.5) (end 25.92 56) (width 0.8) (layer "B.Cu") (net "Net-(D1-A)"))
 (segment (start 25.92 56) (end 30.5 60.58) (width 0.8) (layer "B.Cu") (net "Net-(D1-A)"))
 (segment (start 35.5 56.5) (end 38.04 59.04) (width 0.8) (layer "B.Cu") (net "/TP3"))
 (segment (start 43.5 66.16) (end 41.58 68.08) (width 0.8) (layer "B.Cu") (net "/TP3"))
 (segment (start 41.58 71) (end 45.5 71) (width 0.8) (layer "B.Cu") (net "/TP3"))
 (segment (start 41.5 68) (end 40.84 68) (width 0.8) (layer "B.Cu") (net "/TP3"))
 (segment (start 43.5 60) (end 43.5 66.16) (width 0.8) (layer "B.Cu") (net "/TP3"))
 (segment (start 33.88 56.5) (end 35.5 56.5) (width 0.8) (layer "B.Cu") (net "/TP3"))
 (segment (start 40.84 68) (end 37.84 65) (width 0.8) (layer "B.Cu") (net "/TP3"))
 (segment (start 42.54 59.04) (end 43.5 60) (width 0.8) (layer "B.Cu") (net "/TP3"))
 (segment (start 41.58 68.08) (end 41.58 71) (width 0.8) (layer "B.Cu") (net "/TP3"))
 (segment (start 41.5 59.04) (end 42.54 59.04) (width 0.8) (layer "B.Cu") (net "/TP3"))
 (segment (start 38.04 59.04) (end 41.5 59.04) (width 0.8) (layer "B.Cu") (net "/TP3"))
 (segment (start 46.66 33.5) (end 44.5 33.5) (width 0.8) (layer "B.Cu") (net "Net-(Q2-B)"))
 (segment (start 44.5 33.5) (end 41.49 36.51) (width 0.8) (layer "B.Cu") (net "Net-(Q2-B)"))
 (segment (start 41.49 36.51) (end 41.49 37.95) (width 0.8) (layer "B.Cu") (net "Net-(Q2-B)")))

